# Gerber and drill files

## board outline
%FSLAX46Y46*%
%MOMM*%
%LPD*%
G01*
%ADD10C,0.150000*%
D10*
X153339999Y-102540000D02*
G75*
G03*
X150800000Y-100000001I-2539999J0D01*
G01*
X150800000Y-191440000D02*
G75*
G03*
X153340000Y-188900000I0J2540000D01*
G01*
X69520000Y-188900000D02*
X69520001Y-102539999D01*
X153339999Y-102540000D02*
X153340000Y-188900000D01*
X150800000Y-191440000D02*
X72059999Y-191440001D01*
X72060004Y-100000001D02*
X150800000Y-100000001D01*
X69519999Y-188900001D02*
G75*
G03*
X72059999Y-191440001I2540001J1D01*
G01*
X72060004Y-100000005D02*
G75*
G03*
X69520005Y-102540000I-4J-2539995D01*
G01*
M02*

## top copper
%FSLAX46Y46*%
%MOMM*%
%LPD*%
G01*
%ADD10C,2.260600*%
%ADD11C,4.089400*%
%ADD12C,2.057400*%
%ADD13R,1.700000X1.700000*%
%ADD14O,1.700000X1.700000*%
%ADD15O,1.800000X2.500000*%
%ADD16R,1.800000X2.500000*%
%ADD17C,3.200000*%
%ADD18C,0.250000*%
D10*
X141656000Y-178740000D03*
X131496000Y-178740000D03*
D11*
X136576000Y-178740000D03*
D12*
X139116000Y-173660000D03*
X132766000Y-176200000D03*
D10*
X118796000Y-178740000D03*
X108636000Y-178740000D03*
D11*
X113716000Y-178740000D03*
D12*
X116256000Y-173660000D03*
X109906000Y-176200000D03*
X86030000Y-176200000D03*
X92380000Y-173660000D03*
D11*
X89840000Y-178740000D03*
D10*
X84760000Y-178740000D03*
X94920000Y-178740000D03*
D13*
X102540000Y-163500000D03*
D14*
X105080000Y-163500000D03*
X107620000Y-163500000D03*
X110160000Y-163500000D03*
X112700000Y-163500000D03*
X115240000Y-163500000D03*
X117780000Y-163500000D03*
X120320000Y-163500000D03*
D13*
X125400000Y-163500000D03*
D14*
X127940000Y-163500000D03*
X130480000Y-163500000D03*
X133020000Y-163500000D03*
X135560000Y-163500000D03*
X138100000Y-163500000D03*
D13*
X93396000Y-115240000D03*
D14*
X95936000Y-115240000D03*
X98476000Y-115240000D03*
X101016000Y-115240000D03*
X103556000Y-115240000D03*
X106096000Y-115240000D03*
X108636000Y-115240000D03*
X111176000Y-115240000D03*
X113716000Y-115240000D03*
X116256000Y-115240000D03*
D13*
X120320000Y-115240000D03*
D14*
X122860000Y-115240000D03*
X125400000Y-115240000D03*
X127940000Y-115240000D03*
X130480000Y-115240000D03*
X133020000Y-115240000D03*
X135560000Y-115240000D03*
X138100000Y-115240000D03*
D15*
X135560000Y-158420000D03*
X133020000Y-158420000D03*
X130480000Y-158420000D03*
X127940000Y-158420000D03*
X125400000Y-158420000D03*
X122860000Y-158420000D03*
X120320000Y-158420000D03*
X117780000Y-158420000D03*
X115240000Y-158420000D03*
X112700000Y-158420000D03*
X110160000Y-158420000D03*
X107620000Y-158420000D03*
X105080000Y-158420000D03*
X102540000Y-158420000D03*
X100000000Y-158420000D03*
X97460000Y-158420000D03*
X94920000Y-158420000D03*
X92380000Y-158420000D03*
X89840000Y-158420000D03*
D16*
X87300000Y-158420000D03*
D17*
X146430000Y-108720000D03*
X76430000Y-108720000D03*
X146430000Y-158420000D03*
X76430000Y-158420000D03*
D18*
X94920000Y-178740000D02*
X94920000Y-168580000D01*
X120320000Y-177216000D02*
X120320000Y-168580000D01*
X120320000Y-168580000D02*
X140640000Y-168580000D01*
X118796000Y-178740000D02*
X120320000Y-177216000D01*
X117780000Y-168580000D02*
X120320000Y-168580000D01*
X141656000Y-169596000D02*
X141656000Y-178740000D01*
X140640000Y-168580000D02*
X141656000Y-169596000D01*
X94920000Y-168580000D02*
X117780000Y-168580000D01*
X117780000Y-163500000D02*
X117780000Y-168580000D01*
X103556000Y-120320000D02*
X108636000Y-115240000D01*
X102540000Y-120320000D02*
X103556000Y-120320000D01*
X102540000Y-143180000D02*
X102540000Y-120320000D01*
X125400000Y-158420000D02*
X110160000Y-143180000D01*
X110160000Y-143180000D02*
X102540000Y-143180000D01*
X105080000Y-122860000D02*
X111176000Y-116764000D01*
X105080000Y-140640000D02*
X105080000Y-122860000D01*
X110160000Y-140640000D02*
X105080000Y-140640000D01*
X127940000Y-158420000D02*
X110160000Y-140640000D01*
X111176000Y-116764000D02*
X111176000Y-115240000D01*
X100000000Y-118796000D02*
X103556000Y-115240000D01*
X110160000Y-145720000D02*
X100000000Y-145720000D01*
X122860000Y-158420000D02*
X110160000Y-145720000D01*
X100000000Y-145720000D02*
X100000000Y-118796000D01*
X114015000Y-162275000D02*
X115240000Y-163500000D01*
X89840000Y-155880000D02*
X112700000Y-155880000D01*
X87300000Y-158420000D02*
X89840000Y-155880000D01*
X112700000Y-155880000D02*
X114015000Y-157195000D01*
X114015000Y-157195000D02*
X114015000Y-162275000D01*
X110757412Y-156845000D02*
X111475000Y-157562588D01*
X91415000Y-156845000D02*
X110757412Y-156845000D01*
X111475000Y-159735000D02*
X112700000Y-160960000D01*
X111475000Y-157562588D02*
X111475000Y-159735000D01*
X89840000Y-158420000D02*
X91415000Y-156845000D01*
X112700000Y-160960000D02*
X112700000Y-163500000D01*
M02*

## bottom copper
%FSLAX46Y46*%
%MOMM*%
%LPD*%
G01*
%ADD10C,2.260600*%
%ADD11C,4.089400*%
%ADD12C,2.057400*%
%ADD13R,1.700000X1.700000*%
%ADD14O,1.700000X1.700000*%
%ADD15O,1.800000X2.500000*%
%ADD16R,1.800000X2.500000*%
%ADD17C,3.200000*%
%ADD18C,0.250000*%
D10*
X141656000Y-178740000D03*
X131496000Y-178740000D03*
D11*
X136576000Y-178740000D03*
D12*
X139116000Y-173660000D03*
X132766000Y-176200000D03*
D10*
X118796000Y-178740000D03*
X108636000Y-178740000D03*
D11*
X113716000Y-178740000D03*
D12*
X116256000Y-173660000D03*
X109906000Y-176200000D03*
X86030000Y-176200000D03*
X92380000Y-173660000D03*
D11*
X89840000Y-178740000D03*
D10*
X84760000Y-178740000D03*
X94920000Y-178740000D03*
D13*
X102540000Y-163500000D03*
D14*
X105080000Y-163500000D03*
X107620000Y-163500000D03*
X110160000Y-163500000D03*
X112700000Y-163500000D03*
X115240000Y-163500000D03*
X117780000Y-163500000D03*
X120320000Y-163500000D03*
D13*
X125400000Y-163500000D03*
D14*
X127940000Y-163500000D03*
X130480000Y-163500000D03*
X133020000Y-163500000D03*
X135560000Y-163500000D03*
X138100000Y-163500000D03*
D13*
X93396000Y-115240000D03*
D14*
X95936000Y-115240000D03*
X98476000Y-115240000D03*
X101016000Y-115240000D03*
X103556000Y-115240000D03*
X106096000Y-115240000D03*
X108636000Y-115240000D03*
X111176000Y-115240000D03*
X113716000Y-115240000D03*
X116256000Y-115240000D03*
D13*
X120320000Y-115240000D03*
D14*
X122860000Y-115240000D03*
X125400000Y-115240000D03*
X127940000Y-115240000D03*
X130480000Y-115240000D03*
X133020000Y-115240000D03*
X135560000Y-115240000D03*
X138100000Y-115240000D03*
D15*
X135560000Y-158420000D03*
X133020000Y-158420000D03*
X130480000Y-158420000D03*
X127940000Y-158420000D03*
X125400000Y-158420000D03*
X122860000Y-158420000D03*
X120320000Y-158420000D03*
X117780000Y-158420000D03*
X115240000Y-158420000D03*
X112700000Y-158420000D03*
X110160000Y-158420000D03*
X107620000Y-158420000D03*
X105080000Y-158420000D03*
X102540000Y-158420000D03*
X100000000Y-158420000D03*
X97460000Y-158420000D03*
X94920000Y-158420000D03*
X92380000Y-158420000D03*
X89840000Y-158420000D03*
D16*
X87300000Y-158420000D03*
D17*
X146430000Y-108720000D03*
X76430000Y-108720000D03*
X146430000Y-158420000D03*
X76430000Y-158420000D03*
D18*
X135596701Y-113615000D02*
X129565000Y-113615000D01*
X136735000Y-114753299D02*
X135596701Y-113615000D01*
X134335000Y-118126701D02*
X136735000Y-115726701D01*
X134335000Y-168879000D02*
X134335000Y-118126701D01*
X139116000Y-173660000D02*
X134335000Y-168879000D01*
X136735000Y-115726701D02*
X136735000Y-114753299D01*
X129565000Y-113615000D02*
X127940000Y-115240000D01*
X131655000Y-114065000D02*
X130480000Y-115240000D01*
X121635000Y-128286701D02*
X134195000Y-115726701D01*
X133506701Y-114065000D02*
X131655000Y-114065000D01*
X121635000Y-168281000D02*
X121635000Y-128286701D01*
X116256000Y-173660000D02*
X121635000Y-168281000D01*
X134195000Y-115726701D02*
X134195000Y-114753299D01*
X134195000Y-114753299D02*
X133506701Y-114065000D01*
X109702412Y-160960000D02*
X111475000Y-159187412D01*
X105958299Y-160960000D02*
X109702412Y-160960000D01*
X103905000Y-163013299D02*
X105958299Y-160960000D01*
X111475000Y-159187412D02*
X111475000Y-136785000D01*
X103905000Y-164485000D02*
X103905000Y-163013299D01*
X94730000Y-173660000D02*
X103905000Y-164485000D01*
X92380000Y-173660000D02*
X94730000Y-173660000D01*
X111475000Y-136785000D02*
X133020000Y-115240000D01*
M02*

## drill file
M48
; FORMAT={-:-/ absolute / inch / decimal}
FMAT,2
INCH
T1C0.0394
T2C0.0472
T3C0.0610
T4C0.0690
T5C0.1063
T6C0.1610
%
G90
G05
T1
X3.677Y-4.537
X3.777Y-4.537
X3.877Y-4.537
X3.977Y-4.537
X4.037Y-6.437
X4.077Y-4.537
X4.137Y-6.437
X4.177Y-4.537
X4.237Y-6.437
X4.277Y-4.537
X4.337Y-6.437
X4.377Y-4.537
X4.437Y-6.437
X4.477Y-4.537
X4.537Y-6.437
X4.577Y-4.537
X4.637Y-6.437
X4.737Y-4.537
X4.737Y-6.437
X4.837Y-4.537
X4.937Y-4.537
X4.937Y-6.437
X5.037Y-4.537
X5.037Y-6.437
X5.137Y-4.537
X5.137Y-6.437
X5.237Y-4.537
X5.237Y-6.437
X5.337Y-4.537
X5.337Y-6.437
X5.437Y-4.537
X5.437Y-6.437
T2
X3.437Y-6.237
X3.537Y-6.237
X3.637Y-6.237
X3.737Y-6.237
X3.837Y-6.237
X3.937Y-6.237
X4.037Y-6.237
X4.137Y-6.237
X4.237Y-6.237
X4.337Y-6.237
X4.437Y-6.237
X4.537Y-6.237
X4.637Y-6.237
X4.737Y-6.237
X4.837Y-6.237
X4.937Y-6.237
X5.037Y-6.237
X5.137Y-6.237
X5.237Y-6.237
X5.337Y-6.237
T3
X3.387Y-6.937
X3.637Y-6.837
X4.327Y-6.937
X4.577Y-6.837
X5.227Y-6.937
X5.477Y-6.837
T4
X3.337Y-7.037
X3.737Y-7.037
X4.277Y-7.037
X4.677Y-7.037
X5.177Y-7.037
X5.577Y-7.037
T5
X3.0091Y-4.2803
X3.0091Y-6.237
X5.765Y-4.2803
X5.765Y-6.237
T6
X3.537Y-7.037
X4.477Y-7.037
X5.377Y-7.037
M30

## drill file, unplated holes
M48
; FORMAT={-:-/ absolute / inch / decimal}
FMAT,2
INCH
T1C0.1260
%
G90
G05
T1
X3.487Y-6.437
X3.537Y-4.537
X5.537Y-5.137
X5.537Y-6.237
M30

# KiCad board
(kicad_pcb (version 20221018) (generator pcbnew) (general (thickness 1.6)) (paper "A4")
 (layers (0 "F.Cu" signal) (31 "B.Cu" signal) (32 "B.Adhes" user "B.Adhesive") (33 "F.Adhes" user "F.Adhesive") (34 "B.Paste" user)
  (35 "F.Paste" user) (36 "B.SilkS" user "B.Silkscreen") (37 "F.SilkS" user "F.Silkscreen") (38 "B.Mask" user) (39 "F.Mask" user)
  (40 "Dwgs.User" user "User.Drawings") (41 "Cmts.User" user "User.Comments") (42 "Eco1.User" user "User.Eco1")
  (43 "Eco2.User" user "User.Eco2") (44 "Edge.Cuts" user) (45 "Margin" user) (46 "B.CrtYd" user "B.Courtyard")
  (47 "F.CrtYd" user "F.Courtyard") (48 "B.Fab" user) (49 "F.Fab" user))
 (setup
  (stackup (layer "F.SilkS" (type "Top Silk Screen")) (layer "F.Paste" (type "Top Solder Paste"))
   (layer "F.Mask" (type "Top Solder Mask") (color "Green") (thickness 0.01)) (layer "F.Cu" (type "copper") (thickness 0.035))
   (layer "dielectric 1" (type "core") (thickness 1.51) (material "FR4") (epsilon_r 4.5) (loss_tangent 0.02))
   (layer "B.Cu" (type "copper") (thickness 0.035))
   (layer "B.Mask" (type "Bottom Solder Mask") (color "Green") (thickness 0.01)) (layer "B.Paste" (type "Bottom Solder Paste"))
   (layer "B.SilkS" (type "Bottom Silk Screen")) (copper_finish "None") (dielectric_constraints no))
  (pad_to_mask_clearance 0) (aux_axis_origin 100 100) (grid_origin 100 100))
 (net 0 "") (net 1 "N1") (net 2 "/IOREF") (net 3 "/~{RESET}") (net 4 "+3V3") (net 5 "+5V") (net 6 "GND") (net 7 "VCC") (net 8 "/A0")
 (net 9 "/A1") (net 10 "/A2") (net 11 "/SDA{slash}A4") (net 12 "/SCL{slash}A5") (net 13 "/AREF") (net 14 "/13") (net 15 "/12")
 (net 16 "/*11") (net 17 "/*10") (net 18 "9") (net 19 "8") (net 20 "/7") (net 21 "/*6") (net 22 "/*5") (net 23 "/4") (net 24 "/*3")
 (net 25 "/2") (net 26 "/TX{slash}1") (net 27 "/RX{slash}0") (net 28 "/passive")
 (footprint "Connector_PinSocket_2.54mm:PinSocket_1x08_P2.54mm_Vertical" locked (layer "F.Cu") (at 102.54 163.5 90)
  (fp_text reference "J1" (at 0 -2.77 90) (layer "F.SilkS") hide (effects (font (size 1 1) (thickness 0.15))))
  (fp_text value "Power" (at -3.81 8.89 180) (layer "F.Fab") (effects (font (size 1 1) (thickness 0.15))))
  (pad "1" thru_hole rect locked (at 0 0 90) (size 1.7 1.7) (drill 1) (layers "*.Cu" "*.Mask") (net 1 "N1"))
  (pad "2" thru_hole oval locked (at 0 2.54 90) (size 1.7 1.7) (drill 1) (layers "*.Cu" "*.Mask") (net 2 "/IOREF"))
  (pad "3" thru_hole oval locked (at 0 5.08 90) (size 1.7 1.7) (drill 1) (layers "*.Cu" "*.Mask") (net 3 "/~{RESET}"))
  (pad "4" thru_hole oval locked (at 0 7.62 90) (size 1.7 1.7) (drill 1) (layers "*.Cu" "*.Mask") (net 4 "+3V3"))
  (pad "5" thru_hole oval locked (at 0 10.16 90) (size 1.7 1.7) (drill 1) (layers "*.Cu" "*.Mask") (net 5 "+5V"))
  (pad "6" thru_hole oval locked (at 0 12.7 90) (size 1.7 1.7) (drill 1) (layers "*.Cu" "*.Mask") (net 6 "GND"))
  (pad "7" thru_hole oval locked (at 0 15.24 90) (size 1.7 1.7) (drill 1) (layers "*.Cu" "*.Mask") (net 6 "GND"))
  (pad "8" thru_hole oval locked (at 0 17.78 90) (size 1.7 1.7) (drill 1) (layers "*.Cu" "*.Mask") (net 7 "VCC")))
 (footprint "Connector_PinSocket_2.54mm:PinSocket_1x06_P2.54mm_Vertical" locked (layer "F.Cu") (at 125.4 163.5 90)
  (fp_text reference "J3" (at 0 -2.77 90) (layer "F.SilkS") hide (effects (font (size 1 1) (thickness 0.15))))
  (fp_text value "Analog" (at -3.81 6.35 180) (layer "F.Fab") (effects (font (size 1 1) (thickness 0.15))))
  (pad "1" thru_hole rect locked (at 0 0 90) (size 1.7 1.7) (drill 1) (layers "*.Cu" "*.Mask") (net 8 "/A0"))
  (pad "2" thru_hole oval locked (at 0 2.54 90) (size 1.7 1.7) (drill 1) (layers "*.Cu" "*.Mask") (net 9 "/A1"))
  (pad "3" thru_hole oval locked (at 0 5.08 90) (size 1.7 1.7) (drill 1) (layers "*.Cu" "*.Mask") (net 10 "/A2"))
  (pad "4" thru_hole oval locked (at 0 7.62 90) (size 1.7 1.7) (drill 1) (layers "*.Cu" "*.Mask") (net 6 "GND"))
  (pad "5" thru_hole oval locked (at 0 10.16 90) (size 1.7 1.7) (drill 1) (layers "*.Cu" "*.Mask") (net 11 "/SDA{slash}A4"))
  (pad "6" thru_hole oval locked (at 0 12.7 90) (size 1.7 1.7) (drill 1) (layers "*.Cu" "*.Mask") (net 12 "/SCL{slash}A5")))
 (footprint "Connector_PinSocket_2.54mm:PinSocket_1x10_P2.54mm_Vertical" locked (layer "F.Cu") (at 93.396 115.24 90)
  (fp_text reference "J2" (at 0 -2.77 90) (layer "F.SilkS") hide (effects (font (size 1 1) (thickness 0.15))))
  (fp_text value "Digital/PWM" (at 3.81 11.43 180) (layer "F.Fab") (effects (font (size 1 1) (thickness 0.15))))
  (pad "1" thru_hole rect locked (at 0 0 90) (size 1.7 1.7) (drill 1) (layers "*.Cu" "*.Mask") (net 12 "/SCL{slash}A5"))
  (pad "2" thru_hole oval locked (at 0 2.54 90) (size 1.7 1.7) (drill 1) (layers "*.Cu" "*.Mask") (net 11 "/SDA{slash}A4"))
  (pad "3" thru_hole oval locked (at 0 5.08 90) (size 1.7 1.7) (drill 1) (layers "*.Cu" "*.Mask") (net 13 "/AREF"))
  (pad "4" thru_hole oval locked (at 0 7.62 90) (size 1.7 1.7) (drill 1) (layers "*.Cu" "*.Mask") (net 6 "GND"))
  (pad "5" thru_hole oval locked (at 0 10.16 90) (size 1.7 1.7) (drill 1) (layers "*.Cu" "*.Mask") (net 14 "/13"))
  (pad "6" thru_hole oval locked (at 0 12.7 90) (size 1.7 1.7) (drill 1) (layers "*.Cu" "*.Mask") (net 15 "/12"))
  (pad "7" thru_hole oval locked (at 0 15.24 90) (size 1.7 1.7) (drill 1) (layers "*.Cu" "*.Mask") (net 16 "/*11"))
  (pad "8" thru_hole oval locked (at 0 17.78 90) (size 1.7 1.7) (drill 1) (layers "*.Cu" "*.Mask") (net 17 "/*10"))
  (pad "9" thru_hole oval locked (at 0 20.32 90) (size 1.7 1.7) (drill 1) (layers "*.Cu" "*.Mask") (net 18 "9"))
  (pad "10" thru_hole oval locked (at 0 22.86 90) (size 1.7 1.7) (drill 1) (layers "*.Cu" "*.Mask") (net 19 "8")))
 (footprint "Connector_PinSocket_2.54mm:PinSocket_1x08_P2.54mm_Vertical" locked (layer "F.Cu") (at 120.32 115.24 90)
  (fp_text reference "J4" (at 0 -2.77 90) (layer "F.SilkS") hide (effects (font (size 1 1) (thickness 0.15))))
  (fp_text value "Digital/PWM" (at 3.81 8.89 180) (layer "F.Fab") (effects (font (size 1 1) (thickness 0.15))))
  (pad "1" thru_hole rect locked (at 0 0 90) (size 1.7 1.7) (drill 1) (layers "*.Cu" "*.Mask") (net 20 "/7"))
  (pad "2" thru_hole oval locked (at 0 2.54 90) (size 1.7 1.7) (drill 1) (layers "*.Cu" "*.Mask") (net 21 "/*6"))
  (pad "3" thru_hole oval locked (at 0 5.08 90) (size 1.7 1.7) (drill 1) (layers "*.Cu" "*.Mask") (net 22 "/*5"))
  (pad "4" thru_hole oval locked (at 0 7.62 90) (size 1.7 1.7) (drill 1) (layers "*.Cu" "*.Mask") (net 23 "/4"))
  (pad "5" thru_hole oval locked (at 0 10.16 90) (size 1.7 1.7) (drill 1) (layers "*.Cu" "*.Mask") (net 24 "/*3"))
  (pad "6" thru_hole oval locked (at 0 12.7 90) (size 1.7 1.7) (drill 1) (layers "*.Cu" "*.Mask") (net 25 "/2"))
  (pad "7" thru_hole oval locked (at 0 15.24 90) (size 1.7 1.7) (drill 1) (layers "*.Cu" "*.Mask") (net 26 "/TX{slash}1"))
  (pad "8" thru_hole oval locked (at 0 17.78 90) (size 1.7 1.7) (drill 1) (layers "*.Cu" "*.Mask") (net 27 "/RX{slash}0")))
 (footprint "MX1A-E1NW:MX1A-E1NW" (layer "F.Cu") (at 109.906 176.2)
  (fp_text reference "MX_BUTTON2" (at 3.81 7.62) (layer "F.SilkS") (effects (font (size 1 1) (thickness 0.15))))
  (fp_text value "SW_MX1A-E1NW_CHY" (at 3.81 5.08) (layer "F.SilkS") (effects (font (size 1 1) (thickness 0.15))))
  (pad "1" thru_hole circle (at 0 0) (size 2.0574 2.0574) (drill 1.5494) (layers "*.Cu" "*.Mask"))
  (pad "2" thru_hole circle (at 6.35 -2.54) (size 2.0574 2.0574) (drill 1.5494) (layers "*.Cu" "*.Mask") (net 24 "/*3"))
  (pad "3" thru_hole circle (at 3.81 2.54) (size 4.0894 4.0894) (drill 4.0894) (layers "*.Cu" "*.Mask"))
  (pad "4" thru_hole circle (at -1.27 2.54) (size 2.2606 2.2606) (drill 1.7526) (layers "*.Cu" "*.Mask"))
  (pad "5" thru_hole circle (at 8.89 2.54) (size 2.2606 2.2606) (drill 1.7526) (layers "*.Cu" "*.Mask") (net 6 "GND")))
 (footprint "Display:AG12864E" (layer "F.Cu") (at 87.3 158.42 90)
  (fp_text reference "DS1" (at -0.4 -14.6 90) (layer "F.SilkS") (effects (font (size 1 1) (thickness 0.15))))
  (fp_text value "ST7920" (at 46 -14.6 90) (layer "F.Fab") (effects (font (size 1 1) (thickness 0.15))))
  (pad "" thru_hole circle (at 0 -10.87) (size 3.2 3.2) (drill 2.7) (layers "*.Cu" "*.Mask"))
  (pad "" thru_hole circle (at 0 59.13) (size 3.2 3.2) (drill 2.7) (layers "*.Cu" "*.Mask"))
  (pad "" thru_hole circle (at 49.7 -10.87) (size 3.2 3.2) (drill 2.7) (layers "*.Cu" "*.Mask"))
  (pad "" thru_hole circle (at 49.7 59.13) (size 3.2 3.2) (drill 2.7) (layers "*.Cu" "*.Mask"))
  (pad "1" thru_hole rect (at 0 0) (size 1.8 2.5) (drill 1.2) (layers "*.Cu" "*.Mask") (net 6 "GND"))
  (pad "2" thru_hole oval (at 0 2.54) (size 1.8 2.5) (drill 1.2) (layers "*.Cu" "*.Mask") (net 5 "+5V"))
  (pad "3" thru_hole oval (at 0 5.08) (size 1.8 2.5) (drill 1.2) (layers "*.Cu" "*.Mask") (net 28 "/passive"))
  (pad "4" thru_hole oval (at 0 7.62) (size 1.8 2.5) (drill 1.2) (layers "*.Cu" "*.Mask") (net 28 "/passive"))
  (pad "5" thru_hole oval (at 0 10.16) (size 1.8 2.5) (drill 1.2) (layers "*.Cu" "*.Mask") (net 28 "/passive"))
  (pad "6" thru_hole oval (at 0 12.7) (size 1.8 2.5) (drill 1.2) (layers "*.Cu" "*.Mask") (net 6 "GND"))
  (pad "7" thru_hole oval (at 0 15.24) (size 1.8 2.5) (drill 1.2) (layers "*.Cu" "*.Mask") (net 28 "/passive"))
  (pad "8" thru_hole oval (at 0 17.78) (size 1.8 2.5) (drill 1.2) (layers "*.Cu" "*.Mask") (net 28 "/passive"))
  (pad "9" thru_hole oval (at 0 20.32) (size 1.8 2.5) (drill 1.2) (layers "*.Cu" "*.Mask") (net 28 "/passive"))
  (pad "10" thru_hole oval (at 0 22.86) (size 1.8 2.5) (drill 1.2) (layers "*.Cu" "*.Mask") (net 28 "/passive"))
  (pad "11" thru_hole oval (at 0 25.4) (size 1.8 2.5) (drill 1.2) (layers "*.Cu" "*.Mask") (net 28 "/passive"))
  (pad "12" thru_hole oval (at 0 27.94) (size 1.8 2.5) (drill 1.2) (layers "*.Cu" "*.Mask") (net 28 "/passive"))
  (pad "13" thru_hole oval (at 0 30.48) (size 1.8 2.5) (drill 1.2) (layers "*.Cu" "*.Mask") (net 28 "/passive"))
  (pad "14" thru_hole oval (at 0 33.02) (size 1.8 2.5) (drill 1.2) (layers "*.Cu" "*.Mask") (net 28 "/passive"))
  (pad "15" thru_hole oval (at 0 35.56) (size 1.8 2.5) (drill 1.2) (layers "*.Cu" "*.Mask") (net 14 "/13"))
  (pad "16" thru_hole oval (at 0 38.1) (size 1.8 2.5) (drill 1.2) (layers "*.Cu" "*.Mask") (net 16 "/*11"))
  (pad "17" thru_hole oval (at 0 40.64) (size 1.8 2.5) (drill 1.2) (layers "*.Cu" "*.Mask") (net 17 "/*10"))
  (pad "18" thru_hole oval (at 0 43.18) (size 1.8 2.5) (drill 1.2) (layers "*.Cu" "*.Mask") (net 28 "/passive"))
  (pad "19" thru_hole oval (at 0 45.72) (size 1.8 2.5) (drill 1.2) (layers "*.Cu" "*.Mask") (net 5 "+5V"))
  (pad "20" thru_hole oval (at 0 48.26) (size 1.8 2.5) (drill 1.2) (layers "*.Cu" "*.Mask") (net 6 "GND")))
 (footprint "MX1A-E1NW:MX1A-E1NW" (layer "F.Cu") (at 86.03 176.2)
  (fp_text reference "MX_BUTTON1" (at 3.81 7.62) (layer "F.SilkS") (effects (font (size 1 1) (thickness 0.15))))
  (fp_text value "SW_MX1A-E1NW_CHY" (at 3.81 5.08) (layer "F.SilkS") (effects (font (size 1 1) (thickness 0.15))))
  (pad "1" thru_hole circle (at 0 0) (size 2.0574 2.0574) (drill 1.5494) (layers "*.Cu" "*.Mask"))
  (pad "2" thru_hole circle (at 6.35 -2.54) (size 2.0574 2.0574) (drill 1.5494) (layers "*.Cu" "*.Mask") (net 25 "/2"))
  (pad "3" thru_hole circle (at 3.81 2.54) (size 4.0894 4.0894) (drill 4.0894) (layers "*.Cu" "*.Mask"))
  (pad "4" thru_hole circle (at -1.27 2.54) (size 2.2606 2.2606) (drill 1.7526) (layers "*.Cu" "*.Mask"))
  (pad "5" thru_hole circle (at 8.89 2.54) (size 2.2606 2.2606) (drill 1.7526) (layers "*.Cu" "*.Mask") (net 6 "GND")))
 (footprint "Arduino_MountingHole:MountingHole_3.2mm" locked (layer "F.Cu") (at 89.84 115.24)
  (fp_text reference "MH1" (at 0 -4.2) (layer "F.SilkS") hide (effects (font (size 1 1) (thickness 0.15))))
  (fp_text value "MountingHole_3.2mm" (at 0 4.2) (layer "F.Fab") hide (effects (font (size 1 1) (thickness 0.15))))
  (pad "" np_thru_hole circle locked (at 0 0) (size 3.2 3.2) (drill 3.2) (layers "*.Cu" "*.Mask")))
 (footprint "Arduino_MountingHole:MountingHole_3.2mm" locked (layer "F.Cu") (at 88.57 163.5)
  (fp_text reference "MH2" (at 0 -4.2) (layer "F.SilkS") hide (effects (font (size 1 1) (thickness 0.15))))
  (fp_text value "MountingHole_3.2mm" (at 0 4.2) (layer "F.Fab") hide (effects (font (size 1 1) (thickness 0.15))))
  (pad "" np_thru_hole circle locked (at 0 0) (size 3.2 3.2) (drill 3.2) (layers "*.Cu" "*.Mask")))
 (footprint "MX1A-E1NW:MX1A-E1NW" (layer "F.Cu") (at 132.766 176.2)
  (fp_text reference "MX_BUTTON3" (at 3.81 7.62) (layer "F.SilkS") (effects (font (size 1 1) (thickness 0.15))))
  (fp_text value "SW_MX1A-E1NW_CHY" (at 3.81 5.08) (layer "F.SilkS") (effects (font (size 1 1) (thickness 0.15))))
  (pad "1" thru_hole circle (at 0 0) (size 2.0574 2.0574) (drill 1.5494) (layers "*.Cu" "*.Mask"))
  (pad "2" thru_hole circle (at 6.35 -2.54) (size 2.0574 2.0574) (drill 1.5494) (layers "*.Cu" "*.Mask") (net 23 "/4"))
  (pad "3" thru_hole circle (at 3.81 2.54) (size 4.0894 4.0894) (drill 4.0894) (layers "*.Cu" "*.Mask"))
  (pad "4" thru_hole circle (at -1.27 2.54) (size 2.2606 2.2606) (drill 1.7526) (layers "*.Cu" "*.Mask"))
  (pad "5" thru_hole circle (at 8.89 2.54) (size 2.2606 2.2606) (drill 1.7526) (layers "*.Cu" "*.Mask") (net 6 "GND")))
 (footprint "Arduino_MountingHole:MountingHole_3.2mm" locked (layer "F.Cu") (at 140.64 130.48)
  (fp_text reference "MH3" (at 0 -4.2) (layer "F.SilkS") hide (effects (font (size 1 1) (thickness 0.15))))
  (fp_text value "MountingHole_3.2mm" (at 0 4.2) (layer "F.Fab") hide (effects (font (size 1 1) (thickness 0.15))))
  (pad "" np_thru_hole circle locked (at 0 0) (size 3.2 3.2) (drill 3.2) (layers "*.Cu" "*.Mask")))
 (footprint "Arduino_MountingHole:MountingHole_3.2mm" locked (layer "F.Cu") (at 140.64 158.42)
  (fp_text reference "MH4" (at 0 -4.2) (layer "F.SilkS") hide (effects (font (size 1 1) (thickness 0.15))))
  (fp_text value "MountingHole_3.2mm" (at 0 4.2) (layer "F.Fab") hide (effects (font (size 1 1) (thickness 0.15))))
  (pad "" np_thru_hole circle locked (at 0 0) (size 3.2 3.2) (drill 3.2) (layers "*.Cu" "*.Mask")))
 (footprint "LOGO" (layer "B.Cu") (at 102.54 138.1 90)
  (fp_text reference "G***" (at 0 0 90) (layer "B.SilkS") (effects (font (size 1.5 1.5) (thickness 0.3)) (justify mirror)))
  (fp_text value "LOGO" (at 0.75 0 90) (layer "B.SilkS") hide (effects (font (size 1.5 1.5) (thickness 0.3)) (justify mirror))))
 (gr_arc (start 150.8 100.000001) (mid 152.596051 100.743949) (end 153.339999 102.54) (stroke (width 0.15) (type default))
  (layer "Edge.Cuts"))
 (gr_arc (start 153.34 188.9) (mid 152.596051 190.696051) (end 150.8 191.44) (stroke (width 0.15) (type default)) (layer "Edge.Cuts"))
 (gr_line (start 69.52 188.9) (end 69.520001 102.539999) (stroke (width 0.15) (type solid)) (layer "Edge.Cuts"))
 (gr_line (start 153.339999 102.54) (end 153.34 188.9) (stroke (width 0.15) (type solid)) (layer "Edge.Cuts"))
 (gr_line (start 150.8 191.44) (end 72.059999 191.440001) (stroke (width 0.15) (type solid)) (layer "Edge.Cuts"))
 (gr_line (start 72.060004 100.000001) (end 150.8 100.000001) (stroke (width 0.15) (type solid)) (layer "Edge.Cuts"))
 (gr_arc (start 72.059999 191.440001) (mid 70.263948 190.696052) (end 69.519999 188.900001) (stroke (width 0.15) (type default))
  (layer "Edge.Cuts"))
 (gr_arc (start 69.520005 102.54) (mid 70.263954 100.743951) (end 72.060004 100.000001) (stroke (width 0.15) (type default))
  (layer "Edge.Cuts"))
 (segment (start 112.7 155.88) (end 114.015 157.195) (width 0.25) (layer "F.Cu") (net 6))
 (segment (start 117.78 163.5) (end 117.78 168.58) (width 0.25) (layer "F.Cu") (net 6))
 (segment (start 114.015 157.195) (end 114.015 162.275) (width 0.25) (layer "F.Cu") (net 6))
 (segment (start 114.015 162.275) (end 115.24 163.5) (width 0.25) (layer "F.Cu") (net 6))
 (segment (start 94.92 178.74) (end 94.92 168.58) (width 0.25) (layer "F.Cu") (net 6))
 (segment (start 120.32 168.58) (end 140.64 168.58) (width 0.25) (layer "F.Cu") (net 6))
 (segment (start 94.92 168.58) (end 117.78 168.58) (width 0.25) (layer "F.Cu") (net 6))
 (segment (start 118.796 178.74) (end 120.32 177.216) (width 0.25) (layer "F.Cu") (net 6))
 (segment (start 141.656 169.596) (end 141.656 178.74) (width 0.25) (layer "F.Cu") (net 6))
 (segment (start 89.84 155.88) (end 112.7 155.88) (width 0.25) (layer "F.Cu") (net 6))
 (segment (start 140.64 168.58) (end 141.656 169.596) (width 0.25) (layer "F.Cu") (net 6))
 (segment (start 120.32 177.216) (end 120.32 168.58) (width 0.25) (layer "F.Cu") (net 6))
 (segment (start 87.3 158.42) (end 89.84 155.88) (width 0.25) (layer "F.Cu") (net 6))
 (segment (start 117.78 168.58) (end 120.32 168.58) (width 0.25) (layer "F.Cu") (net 6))
 (segment (start 112.7 160.96) (end 112.7 163.5) (width 0.25) (layer "F.Cu") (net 5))
 (segment (start 89.84 158.42) (end 91.415 156.845) (width 0.25) (layer "F.Cu") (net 5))
 (segment (start 111.475 157.562588) (end 111.475 159.735) (width 0.25) (layer "F.Cu") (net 5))
 (segment (start 111.475 159.735) (end 112.7 160.96) (width 0.25) (layer "F.Cu") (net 5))
 (segment (start 91.415 156.845) (end 110.757412 156.845) (width 0.25) (layer "F.Cu") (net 5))
 (segment (start 110.757412 156.845) (end 111.475 157.562588) (width 0.25) (layer "F.Cu") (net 5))
 (segment (start 110.16 145.72) (end 100 145.72) (width 0.25) (layer "F.Cu") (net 14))
 (segment (start 100 118.796) (end 103.556 115.24) (width 0.25) (layer "F.Cu") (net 14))
 (segment (start 122.86 158.42) (end 110.16 145.72) (width 0.25) (layer "F.Cu") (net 14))
 (segment (start 100 145.72) (end 100 118.796) (width 0.25) (layer "F.Cu") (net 14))
 (segment (start 125.4 158.42) (end 110.16 143.18) (width 0.25) (layer "F.Cu") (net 16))
 (segment (start 110.16 143.18) (end 102.54 143.18) (width 0.25) (layer "F.Cu") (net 16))
 (segment (start 102.54 143.18) (end 102.54 120.32) (width 0.25) (layer "F.Cu") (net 16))
 (segment (start 103.556 120.32) (end 108.636 115.24) (width 0.25) (layer "F.Cu") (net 16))
 (segment (start 102.54 120.32) (end 103.556 120.32) (width 0.25) (layer "F.Cu") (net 16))
 (segment (start 110.16 140.64) (end 105.08 140.64) (width 0.25) (layer "F.Cu") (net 17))
 (segment (start 111.176 116.764) (end 111.176 115.24) (width 0.25) (layer "F.Cu") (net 17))
 (segment (start 105.08 122.86) (end 111.176 116.764) (width 0.25) (layer "F.Cu") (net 17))
 (segment (start 105.08 140.64) (end 105.08 122.86) (width 0.25) (layer "F.Cu") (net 17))
 (segment (start 127.94 158.42) (end 110.16 140.64) (width 0.25) (layer "F.Cu") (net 17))
 (segment (start 134.335 168.879) (end 134.335 118.126701) (width 0.25) (layer "B.Cu") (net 23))
 (segment (start 136.735 114.753299) (end 135.596701 113.615) (width 0.25) (layer "B.Cu") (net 23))
 (segment (start 129.565 113.615) (end 127.94 115.24) (width 0.25) (layer "B.Cu") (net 23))
 (segment (start 134.335 118.126701) (end 136.735 115.726701) (width 0.25) (layer "B.Cu") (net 23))
 (segment (start 136.735 115.726701) (end 136.735 114.753299) (width 0.25) (layer "B.Cu") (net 23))
 (segment (start 139.116 173.66) (end 134.335 168.879) (width 0.25) (layer "B.Cu") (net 23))
 (segment (start 135.596701 113.615) (end 129.565 113.615) (width 0.25) (layer "B.Cu") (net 23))
 (segment (start 105.958299 160.96) (end 109.702412 160.96) (width 0.25) (layer "B.Cu") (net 25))
 (segment (start 111.475 136.785) (end 133.02 115.24) (width 0.25) (layer "B.Cu") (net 25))
 (segment (start 94.73 173.66) (end 103.905 164.485) (width 0.25) (layer "B.Cu") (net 25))
 (segment (start 92.38 173.66) (end 94.73 173.66) (width 0.25) (layer "B.Cu") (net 25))
 (segment (start 111.475 159.187412) (end 111.475 136.785) (width 0.25) (layer "B.Cu") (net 25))
 (segment (start 109.702412 160.96) (end 111.475 159.187412) (width 0.25) (layer "B.Cu") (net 25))
 (segment (start 103.905 163.013299) (end 105.958299 160.96) (width 0.25) (layer "B.Cu") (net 25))
 (segment (start 103.905 164.485) (end 103.905 163.013299) (width 0.25) (layer "B.Cu") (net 25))
 (segment (start 116.256 173.66) (end 121.635 168.281) (width 0.25) (layer "B.Cu") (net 24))
 (segment (start 131.655 114.065) (end 130.48 115.24) (width 0.25) (layer "B.Cu") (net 24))
 (segment (start 134.195 115.726701) (end 134.195 114.753299) (width 0.25) (layer "B.Cu") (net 24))
 (segment (start 121.635 128.286701) (end 134.195 115.726701) (width 0.25) (layer "B.Cu") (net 24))
 (segment (start 134.195 114.753299) (end 133.506701 114.065) (width 0.25) (layer "B.Cu") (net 24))
 (segment (start 121.635 168.281) (end 121.635 128.286701) (width 0.25) (layer "B.Cu") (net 24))
 (segment (start 133.506701 114.065) (end 131.655 114.065) (width 0.25) (layer "B.Cu") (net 24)))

